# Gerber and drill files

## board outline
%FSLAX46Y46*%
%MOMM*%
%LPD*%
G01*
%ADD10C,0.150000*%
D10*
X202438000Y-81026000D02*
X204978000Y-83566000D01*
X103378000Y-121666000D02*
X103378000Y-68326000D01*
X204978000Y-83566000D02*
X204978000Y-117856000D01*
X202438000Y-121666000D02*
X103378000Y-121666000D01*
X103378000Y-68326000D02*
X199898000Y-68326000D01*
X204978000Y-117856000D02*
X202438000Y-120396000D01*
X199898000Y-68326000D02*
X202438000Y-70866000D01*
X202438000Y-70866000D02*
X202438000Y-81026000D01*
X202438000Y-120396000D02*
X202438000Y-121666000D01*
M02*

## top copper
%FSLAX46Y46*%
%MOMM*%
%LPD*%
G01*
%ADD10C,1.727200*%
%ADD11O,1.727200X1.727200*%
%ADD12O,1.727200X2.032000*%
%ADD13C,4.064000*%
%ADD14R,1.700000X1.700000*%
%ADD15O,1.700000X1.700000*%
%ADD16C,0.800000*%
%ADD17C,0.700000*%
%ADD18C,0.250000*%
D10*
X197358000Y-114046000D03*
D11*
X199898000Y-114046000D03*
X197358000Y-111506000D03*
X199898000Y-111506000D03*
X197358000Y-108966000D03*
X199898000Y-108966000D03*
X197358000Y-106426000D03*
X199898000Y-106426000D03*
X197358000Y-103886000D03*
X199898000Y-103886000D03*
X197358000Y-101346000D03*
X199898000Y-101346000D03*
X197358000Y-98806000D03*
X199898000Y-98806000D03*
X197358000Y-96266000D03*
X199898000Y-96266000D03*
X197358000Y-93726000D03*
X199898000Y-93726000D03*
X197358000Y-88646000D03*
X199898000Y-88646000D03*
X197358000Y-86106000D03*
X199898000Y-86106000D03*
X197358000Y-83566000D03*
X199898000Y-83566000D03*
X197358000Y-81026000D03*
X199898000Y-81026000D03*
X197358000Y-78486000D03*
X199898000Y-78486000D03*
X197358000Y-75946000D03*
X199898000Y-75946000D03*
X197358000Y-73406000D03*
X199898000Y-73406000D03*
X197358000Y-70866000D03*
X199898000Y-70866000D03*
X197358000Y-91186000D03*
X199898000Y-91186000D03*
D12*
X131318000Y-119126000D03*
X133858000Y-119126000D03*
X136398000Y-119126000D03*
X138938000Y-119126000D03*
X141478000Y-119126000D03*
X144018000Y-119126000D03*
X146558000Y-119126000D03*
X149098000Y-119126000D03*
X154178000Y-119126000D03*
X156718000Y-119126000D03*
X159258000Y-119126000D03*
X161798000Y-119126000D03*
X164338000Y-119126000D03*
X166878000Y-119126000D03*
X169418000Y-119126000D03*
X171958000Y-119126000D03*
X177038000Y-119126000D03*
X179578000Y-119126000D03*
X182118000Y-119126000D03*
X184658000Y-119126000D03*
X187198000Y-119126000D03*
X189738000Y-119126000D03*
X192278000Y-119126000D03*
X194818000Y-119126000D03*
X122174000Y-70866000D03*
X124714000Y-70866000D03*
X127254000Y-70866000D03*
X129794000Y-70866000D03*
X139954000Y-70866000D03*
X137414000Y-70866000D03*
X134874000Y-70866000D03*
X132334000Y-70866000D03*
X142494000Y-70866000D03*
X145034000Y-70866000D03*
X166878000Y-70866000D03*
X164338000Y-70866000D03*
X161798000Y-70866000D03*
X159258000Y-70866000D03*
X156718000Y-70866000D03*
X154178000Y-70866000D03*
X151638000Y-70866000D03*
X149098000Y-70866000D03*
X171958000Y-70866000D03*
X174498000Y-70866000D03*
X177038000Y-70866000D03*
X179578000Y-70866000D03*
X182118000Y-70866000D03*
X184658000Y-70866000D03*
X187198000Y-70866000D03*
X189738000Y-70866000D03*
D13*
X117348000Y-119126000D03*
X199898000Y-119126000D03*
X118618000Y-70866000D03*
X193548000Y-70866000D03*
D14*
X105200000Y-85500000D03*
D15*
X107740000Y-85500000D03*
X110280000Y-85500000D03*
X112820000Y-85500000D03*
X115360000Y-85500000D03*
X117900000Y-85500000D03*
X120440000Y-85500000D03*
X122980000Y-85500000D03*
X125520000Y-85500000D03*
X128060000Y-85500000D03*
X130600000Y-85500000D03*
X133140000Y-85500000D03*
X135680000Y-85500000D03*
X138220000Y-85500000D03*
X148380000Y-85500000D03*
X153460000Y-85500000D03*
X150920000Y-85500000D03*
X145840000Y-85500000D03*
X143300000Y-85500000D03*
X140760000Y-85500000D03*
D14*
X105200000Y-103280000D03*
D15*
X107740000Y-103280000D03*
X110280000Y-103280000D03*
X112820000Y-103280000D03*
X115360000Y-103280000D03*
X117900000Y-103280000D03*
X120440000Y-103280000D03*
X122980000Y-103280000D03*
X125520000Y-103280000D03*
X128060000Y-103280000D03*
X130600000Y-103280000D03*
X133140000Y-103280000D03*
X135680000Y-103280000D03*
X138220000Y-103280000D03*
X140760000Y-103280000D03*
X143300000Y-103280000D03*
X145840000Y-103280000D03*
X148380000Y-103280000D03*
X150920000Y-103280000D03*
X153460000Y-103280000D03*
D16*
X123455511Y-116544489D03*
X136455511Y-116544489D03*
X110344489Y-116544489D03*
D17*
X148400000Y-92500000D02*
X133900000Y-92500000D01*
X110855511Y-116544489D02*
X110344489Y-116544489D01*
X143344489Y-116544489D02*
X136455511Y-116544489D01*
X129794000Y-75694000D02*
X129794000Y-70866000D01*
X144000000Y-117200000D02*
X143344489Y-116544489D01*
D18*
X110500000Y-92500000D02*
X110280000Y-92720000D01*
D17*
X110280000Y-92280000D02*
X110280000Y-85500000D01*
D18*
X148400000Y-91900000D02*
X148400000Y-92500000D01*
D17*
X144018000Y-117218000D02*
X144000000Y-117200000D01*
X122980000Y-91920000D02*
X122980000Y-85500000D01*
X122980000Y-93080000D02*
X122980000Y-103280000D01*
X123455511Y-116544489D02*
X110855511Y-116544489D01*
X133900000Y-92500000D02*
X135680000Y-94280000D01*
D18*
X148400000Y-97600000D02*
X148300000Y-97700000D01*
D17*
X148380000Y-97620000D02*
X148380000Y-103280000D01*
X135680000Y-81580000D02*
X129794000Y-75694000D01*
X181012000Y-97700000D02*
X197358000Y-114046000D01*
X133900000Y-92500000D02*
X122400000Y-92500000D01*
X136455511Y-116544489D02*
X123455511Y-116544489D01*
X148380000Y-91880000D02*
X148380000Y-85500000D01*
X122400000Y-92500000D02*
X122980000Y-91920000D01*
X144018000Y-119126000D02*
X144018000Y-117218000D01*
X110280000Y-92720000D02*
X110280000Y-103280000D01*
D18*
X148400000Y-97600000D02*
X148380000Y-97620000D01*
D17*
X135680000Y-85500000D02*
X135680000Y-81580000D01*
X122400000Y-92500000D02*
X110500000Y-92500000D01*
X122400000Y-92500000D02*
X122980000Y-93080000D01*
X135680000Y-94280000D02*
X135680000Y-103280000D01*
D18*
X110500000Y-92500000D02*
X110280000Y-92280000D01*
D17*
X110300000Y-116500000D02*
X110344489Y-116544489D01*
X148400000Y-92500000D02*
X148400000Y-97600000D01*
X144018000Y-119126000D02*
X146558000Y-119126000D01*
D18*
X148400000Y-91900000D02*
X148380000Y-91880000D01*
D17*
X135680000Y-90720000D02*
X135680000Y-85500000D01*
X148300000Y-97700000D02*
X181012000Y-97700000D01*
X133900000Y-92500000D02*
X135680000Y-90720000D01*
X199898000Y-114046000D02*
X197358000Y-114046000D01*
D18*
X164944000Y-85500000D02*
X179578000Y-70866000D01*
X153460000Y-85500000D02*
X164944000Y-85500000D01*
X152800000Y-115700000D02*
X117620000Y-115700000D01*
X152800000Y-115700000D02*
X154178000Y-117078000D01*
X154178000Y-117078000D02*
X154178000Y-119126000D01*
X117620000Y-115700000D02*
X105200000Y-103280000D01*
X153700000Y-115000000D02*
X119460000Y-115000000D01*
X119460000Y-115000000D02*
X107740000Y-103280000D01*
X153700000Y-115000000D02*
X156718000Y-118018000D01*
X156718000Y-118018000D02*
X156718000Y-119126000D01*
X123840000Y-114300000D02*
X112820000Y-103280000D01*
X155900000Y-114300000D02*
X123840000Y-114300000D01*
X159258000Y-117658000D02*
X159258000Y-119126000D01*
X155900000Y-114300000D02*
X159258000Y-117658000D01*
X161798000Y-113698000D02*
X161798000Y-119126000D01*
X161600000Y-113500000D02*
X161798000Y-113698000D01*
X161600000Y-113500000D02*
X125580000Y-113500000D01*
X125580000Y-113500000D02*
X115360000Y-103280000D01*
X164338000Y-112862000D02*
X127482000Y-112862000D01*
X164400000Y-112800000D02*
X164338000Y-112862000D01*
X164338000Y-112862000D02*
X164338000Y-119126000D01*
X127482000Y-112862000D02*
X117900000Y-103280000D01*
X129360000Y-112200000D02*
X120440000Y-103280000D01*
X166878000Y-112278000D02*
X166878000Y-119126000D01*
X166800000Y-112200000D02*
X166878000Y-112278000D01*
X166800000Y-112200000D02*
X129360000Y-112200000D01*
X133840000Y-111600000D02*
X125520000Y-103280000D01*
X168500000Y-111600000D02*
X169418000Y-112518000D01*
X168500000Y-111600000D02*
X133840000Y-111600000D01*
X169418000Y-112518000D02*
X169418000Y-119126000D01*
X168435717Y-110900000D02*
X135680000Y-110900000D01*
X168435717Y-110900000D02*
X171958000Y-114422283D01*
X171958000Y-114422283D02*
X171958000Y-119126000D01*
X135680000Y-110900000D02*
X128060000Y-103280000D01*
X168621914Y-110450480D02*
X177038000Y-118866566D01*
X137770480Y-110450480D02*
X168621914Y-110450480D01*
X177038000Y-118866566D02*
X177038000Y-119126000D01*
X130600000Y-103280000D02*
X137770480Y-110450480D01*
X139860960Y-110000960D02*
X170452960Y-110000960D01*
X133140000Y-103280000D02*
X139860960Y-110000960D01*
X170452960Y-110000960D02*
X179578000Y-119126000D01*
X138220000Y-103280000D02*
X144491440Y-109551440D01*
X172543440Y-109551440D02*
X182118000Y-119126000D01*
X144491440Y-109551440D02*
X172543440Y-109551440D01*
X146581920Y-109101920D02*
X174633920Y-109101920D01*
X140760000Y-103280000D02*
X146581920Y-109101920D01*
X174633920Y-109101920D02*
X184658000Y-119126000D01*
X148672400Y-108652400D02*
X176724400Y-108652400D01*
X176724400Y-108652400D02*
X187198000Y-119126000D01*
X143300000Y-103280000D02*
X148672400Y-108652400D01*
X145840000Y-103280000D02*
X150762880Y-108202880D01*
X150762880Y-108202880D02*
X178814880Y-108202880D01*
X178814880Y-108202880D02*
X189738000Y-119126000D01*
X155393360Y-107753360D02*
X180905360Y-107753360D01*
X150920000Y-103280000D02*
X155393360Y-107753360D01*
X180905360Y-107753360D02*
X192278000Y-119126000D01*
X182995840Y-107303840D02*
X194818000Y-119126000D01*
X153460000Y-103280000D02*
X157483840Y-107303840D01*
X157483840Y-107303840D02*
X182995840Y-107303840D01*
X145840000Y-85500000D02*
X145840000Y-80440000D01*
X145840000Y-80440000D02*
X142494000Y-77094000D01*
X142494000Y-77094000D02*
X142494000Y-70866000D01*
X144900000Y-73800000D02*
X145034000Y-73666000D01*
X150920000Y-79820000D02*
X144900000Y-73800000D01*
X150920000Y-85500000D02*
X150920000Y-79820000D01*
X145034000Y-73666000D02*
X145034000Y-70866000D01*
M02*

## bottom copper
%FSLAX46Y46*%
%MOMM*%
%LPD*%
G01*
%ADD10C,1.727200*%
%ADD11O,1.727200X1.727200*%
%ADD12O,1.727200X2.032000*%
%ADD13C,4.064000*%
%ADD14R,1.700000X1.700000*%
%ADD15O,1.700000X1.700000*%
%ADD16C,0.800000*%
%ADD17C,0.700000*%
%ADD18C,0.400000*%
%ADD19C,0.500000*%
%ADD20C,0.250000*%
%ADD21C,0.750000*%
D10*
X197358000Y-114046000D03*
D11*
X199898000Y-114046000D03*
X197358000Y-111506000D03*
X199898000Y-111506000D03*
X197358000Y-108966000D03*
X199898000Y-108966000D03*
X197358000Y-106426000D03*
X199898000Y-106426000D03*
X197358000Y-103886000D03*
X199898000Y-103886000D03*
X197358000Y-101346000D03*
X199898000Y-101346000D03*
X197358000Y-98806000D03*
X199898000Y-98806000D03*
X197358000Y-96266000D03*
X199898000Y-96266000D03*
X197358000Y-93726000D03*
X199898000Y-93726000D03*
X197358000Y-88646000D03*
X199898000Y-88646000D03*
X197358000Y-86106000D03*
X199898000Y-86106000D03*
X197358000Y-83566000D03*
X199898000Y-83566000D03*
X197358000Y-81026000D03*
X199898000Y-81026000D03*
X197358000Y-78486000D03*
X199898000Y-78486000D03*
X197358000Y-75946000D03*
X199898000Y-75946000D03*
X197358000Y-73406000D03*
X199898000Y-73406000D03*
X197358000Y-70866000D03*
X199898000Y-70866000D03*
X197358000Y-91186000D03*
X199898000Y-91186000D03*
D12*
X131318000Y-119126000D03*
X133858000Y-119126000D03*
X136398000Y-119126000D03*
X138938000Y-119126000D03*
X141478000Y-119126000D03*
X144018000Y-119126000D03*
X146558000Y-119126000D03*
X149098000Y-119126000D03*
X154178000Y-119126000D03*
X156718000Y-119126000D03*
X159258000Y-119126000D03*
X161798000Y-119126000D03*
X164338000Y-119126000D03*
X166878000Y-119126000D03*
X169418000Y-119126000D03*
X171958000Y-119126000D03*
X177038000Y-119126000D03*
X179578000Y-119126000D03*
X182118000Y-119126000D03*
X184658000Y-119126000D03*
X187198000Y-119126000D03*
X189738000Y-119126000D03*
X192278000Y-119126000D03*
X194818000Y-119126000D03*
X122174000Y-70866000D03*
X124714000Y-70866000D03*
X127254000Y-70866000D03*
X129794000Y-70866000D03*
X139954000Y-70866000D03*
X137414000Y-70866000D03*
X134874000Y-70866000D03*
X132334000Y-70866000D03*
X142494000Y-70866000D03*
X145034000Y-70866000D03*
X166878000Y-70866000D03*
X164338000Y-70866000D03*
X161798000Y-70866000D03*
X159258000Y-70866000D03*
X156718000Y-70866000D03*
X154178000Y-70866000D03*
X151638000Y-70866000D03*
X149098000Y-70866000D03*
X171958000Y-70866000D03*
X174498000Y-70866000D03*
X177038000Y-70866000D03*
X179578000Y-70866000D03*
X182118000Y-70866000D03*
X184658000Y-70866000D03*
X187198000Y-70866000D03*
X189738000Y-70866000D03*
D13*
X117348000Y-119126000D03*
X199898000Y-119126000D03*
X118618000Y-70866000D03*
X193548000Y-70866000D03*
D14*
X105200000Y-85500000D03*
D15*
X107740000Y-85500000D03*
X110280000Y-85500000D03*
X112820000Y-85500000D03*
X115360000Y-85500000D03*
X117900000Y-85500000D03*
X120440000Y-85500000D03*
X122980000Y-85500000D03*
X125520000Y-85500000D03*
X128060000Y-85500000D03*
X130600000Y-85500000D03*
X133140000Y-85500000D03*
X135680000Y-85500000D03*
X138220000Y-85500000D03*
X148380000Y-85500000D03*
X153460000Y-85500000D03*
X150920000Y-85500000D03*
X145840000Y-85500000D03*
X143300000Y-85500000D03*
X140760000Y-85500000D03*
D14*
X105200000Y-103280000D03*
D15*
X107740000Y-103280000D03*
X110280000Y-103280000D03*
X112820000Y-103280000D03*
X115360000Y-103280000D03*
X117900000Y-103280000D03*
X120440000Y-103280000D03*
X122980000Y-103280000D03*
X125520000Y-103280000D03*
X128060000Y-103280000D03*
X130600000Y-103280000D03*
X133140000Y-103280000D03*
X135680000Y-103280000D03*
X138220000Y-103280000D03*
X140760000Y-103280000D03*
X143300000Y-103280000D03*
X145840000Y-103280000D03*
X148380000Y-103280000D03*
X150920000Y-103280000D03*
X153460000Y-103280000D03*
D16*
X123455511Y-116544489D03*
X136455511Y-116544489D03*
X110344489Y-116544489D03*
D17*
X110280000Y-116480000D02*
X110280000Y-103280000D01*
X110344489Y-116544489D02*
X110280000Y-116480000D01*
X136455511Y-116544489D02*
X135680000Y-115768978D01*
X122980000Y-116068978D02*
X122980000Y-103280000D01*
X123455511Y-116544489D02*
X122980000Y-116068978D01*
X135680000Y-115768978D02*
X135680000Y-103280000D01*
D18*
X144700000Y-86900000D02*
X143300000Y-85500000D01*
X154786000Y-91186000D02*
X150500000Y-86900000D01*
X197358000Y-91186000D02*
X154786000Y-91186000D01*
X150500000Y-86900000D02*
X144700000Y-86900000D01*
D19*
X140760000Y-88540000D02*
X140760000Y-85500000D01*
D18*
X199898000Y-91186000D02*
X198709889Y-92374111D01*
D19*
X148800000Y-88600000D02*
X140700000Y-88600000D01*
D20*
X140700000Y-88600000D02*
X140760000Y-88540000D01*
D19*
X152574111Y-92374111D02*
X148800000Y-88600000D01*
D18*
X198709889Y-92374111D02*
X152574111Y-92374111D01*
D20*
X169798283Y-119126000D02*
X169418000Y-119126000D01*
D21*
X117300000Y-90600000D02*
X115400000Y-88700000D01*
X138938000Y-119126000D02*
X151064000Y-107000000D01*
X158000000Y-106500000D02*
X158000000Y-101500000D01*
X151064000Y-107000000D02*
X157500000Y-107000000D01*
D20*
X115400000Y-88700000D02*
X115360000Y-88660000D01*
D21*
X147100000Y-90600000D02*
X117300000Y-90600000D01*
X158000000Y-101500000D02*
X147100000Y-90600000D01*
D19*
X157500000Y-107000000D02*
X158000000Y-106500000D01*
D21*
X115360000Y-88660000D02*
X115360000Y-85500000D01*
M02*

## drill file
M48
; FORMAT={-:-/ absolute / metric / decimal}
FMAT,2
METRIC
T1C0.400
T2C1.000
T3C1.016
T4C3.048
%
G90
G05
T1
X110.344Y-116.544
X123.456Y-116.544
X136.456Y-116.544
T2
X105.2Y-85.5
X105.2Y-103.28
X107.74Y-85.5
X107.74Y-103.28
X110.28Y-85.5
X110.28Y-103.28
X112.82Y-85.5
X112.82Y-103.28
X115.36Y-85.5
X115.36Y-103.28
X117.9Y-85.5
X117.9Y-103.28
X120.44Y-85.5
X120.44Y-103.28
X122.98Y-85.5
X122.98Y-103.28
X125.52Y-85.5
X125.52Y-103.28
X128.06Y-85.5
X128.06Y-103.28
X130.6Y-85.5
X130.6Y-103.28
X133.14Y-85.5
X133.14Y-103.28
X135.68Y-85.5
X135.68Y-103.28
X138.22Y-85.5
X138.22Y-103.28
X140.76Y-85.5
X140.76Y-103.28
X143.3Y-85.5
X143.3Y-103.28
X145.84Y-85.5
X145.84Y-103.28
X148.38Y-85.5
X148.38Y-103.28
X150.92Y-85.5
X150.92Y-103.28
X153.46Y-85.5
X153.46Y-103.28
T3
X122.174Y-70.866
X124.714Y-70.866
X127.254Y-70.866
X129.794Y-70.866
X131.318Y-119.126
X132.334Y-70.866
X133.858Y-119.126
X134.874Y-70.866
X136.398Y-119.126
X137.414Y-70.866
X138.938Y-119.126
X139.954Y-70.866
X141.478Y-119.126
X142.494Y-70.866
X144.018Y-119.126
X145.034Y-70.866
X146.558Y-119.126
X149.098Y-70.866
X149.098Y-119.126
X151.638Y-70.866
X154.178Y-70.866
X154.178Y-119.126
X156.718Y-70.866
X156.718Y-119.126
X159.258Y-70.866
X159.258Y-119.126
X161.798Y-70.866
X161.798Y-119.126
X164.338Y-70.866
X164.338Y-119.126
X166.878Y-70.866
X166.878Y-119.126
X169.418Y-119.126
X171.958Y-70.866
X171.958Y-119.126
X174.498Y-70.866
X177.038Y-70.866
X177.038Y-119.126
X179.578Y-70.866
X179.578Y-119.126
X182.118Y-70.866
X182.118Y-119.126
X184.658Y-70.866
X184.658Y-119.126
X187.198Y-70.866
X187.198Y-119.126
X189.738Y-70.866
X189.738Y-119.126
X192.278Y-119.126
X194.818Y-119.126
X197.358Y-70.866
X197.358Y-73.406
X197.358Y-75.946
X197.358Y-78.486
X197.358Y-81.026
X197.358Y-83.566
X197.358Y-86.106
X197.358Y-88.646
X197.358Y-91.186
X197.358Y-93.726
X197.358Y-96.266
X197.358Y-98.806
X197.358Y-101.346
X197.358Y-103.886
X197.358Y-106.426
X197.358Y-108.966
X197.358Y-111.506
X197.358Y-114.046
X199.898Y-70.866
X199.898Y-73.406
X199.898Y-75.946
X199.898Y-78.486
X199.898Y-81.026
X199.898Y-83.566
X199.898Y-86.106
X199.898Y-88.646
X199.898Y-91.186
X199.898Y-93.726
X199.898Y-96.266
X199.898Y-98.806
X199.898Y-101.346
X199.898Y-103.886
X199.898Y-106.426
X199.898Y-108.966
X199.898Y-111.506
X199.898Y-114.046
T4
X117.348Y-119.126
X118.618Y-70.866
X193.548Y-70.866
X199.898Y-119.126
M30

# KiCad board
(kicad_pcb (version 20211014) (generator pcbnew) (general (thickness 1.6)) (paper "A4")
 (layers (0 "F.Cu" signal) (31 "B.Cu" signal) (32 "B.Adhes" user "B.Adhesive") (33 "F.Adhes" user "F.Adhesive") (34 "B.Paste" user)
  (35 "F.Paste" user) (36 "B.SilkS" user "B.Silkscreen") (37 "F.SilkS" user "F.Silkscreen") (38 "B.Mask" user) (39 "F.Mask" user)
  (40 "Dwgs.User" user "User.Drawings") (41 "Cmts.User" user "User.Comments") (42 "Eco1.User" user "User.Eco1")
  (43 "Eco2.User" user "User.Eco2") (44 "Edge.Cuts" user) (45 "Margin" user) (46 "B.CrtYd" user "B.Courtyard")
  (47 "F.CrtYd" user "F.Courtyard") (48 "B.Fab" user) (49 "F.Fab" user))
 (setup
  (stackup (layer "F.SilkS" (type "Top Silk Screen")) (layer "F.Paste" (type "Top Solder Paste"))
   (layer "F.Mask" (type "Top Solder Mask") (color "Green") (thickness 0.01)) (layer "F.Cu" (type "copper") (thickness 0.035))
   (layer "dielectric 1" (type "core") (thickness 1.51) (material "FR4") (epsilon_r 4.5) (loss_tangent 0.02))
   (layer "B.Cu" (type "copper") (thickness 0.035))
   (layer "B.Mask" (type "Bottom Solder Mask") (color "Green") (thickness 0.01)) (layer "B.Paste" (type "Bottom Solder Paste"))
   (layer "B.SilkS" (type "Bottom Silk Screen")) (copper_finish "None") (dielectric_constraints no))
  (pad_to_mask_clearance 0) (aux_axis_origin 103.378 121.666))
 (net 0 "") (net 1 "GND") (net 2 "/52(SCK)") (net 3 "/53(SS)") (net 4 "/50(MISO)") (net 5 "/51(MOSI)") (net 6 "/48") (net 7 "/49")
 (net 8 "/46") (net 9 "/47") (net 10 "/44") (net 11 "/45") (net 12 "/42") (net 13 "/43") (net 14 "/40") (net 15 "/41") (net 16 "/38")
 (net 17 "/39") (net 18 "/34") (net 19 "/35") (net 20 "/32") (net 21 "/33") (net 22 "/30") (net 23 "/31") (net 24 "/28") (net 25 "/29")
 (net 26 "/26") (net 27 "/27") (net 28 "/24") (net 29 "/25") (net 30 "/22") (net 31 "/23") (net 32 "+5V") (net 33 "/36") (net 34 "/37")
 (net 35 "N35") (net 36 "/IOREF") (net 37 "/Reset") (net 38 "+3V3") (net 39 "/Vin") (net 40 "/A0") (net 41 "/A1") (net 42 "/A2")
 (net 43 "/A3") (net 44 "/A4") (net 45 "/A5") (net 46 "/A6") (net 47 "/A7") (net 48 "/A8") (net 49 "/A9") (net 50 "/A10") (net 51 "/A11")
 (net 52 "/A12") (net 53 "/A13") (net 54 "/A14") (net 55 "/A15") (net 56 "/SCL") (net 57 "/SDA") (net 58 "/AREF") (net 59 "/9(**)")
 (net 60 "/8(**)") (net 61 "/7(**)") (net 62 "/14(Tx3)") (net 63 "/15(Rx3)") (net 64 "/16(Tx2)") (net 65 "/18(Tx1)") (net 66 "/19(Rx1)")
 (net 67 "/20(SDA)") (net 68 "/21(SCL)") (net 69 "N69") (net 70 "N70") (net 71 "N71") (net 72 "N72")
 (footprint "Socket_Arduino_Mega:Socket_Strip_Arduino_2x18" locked (layer "F.Cu") (at 197.358 114.046 90)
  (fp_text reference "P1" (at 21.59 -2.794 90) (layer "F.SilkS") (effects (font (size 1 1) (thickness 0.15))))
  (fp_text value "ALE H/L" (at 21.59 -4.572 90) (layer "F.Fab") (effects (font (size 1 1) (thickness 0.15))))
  (pad "1" thru_hole circle locked (at 0 0 90) (size 1.7272 1.7272) (drill 1.016) (layers *.Cu *.Mask "F.SilkS") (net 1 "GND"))
  (pad "2" thru_hole oval locked (at 0 2.54 90) (size 1.7272 1.7272) (drill 1.016) (layers *.Cu *.Mask "F.SilkS") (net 1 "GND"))
  (pad "3" thru_hole oval locked (at 2.54 0 90) (size 1.7272 1.7272) (drill 1.016) (layers *.Cu *.Mask "F.SilkS") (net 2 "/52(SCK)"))
  (pad "4" thru_hole oval locked (at 2.54 2.54 90) (size 1.7272 1.7272) (drill 1.016) (layers *.Cu *.Mask "F.SilkS") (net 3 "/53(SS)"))
  (pad "5" thru_hole oval locked (at 5.08 0 90) (size 1.7272 1.7272) (drill 1.016) (layers *.Cu *.Mask "F.SilkS") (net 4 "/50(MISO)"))
  (pad "6" thru_hole oval locked (at 5.08 2.54 90) (size 1.7272 1.7272) (drill 1.016) (layers *.Cu *.Mask "F.SilkS") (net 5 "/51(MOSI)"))
  (pad "7" thru_hole oval locked (at 7.62 0 90) (size 1.7272 1.7272) (drill 1.016) (layers *.Cu *.Mask "F.SilkS") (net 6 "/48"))
  (pad "8" thru_hole oval locked (at 7.62 2.54 90) (size 1.7272 1.7272) (drill 1.016) (layers *.Cu *.Mask "F.SilkS") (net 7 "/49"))
  (pad "9" thru_hole oval locked (at 10.16 0 90) (size 1.7272 1.7272) (drill 1.016) (layers *.Cu *.Mask "F.SilkS") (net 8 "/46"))
  (pad "10" thru_hole oval locked (at 10.16 2.54 90) (size 1.7272 1.7272) (drill 1.016) (layers *.Cu *.Mask "F.SilkS") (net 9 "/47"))
  (pad "11" thru_hole oval locked (at 12.7 0 90) (size 1.7272 1.7272) (drill 1.016) (layers *.Cu *.Mask "F.SilkS") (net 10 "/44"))
  (pad "12" thru_hole oval locked (at 12.7 2.54 90) (size 1.7272 1.7272) (drill 1.016) (layers *.Cu *.Mask "F.SilkS") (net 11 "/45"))
  (pad "13" thru_hole oval locked (at 15.24 0 90) (size 1.7272 1.7272) (drill 1.016) (layers *.Cu *.Mask "F.SilkS") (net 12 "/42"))
  (pad "14" thru_hole oval locked (at 15.24 2.54 90) (size 1.7272 1.7272) (drill 1.016) (layers *.Cu *.Mask "F.SilkS") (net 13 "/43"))
  (pad "15" thru_hole oval locked (at 17.78 0 90) (size 1.7272 1.7272) (drill 1.016) (layers *.Cu *.Mask "F.SilkS") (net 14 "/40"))
  (pad "16" thru_hole oval locked (at 17.78 2.54 90) (size 1.7272 1.7272) (drill 1.016) (layers *.Cu *.Mask "F.SilkS") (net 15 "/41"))
  (pad "17" thru_hole oval locked (at 20.32 0 90) (size 1.7272 1.7272) (drill 1.016) (layers *.Cu *.Mask "F.SilkS") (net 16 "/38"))
  (pad "18" thru_hole oval locked (at 20.32 2.54 90) (size 1.7272 1.7272) (drill 1.016) (layers *.Cu *.Mask "F.SilkS") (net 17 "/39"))
  (pad "21" thru_hole oval locked (at 25.4 0 90) (size 1.7272 1.7272) (drill 1.016) (layers *.Cu *.Mask "F.SilkS") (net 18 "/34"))
  (pad "22" thru_hole oval locked (at 25.4 2.54 90) (size 1.7272 1.7272) (drill 1.016) (layers *.Cu *.Mask "F.SilkS") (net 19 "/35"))
  (pad "23" thru_hole oval locked (at 27.94 0 90) (size 1.7272 1.7272) (drill 1.016) (layers *.Cu *.Mask "F.SilkS") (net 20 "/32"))
  (pad "24" thru_hole oval locked (at 27.94 2.54 90) (size 1.7272 1.7272) (drill 1.016) (layers *.Cu *.Mask "F.SilkS") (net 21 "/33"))
  (pad "25" thru_hole oval locked (at 30.48 0 90) (size 1.7272 1.7272) (drill 1.016) (layers *.Cu *.Mask "F.SilkS") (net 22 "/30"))
  (pad "26" thru_hole oval locked (at 30.48 2.54 90) (size 1.7272 1.7272) (drill 1.016) (layers *.Cu *.Mask "F.SilkS") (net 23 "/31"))
  (pad "27" thru_hole oval locked (at 33.02 0 90) (size 1.7272 1.7272) (drill 1.016) (layers *.Cu *.Mask "F.SilkS") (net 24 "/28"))
  (pad "28" thru_hole oval locked (at 33.02 2.54 90) (size 1.7272 1.7272) (drill 1.016) (layers *.Cu *.Mask "F.SilkS") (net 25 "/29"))
  (pad "29" thru_hole oval locked (at 35.56 0 90) (size 1.7272 1.7272) (drill 1.016) (layers *.Cu *.Mask "F.SilkS") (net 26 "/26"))
  (pad "30" thru_hole oval locked (at 35.56 2.54 90) (size 1.7272 1.7272) (drill 1.016) (layers *.Cu *.Mask "F.SilkS") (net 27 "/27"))
  (pad "31" thru_hole oval locked (at 38.1 0 90) (size 1.7272 1.7272) (drill 1.016) (layers *.Cu *.Mask "F.SilkS") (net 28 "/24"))
  (pad "32" thru_hole oval locked (at 38.1 2.54 90) (size 1.7272 1.7272) (drill 1.016) (layers *.Cu *.Mask "F.SilkS") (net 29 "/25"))
  (pad "33" thru_hole oval locked (at 40.64 0 90) (size 1.7272 1.7272) (drill 1.016) (layers *.Cu *.Mask "F.SilkS") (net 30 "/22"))
  (pad "34" thru_hole oval locked (at 40.64 2.54 90) (size 1.7272 1.7272) (drill 1.016) (layers *.Cu *.Mask "F.SilkS") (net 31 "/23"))
  (pad "35" thru_hole oval locked (at 43.18 0 90) (size 1.7272 1.7272) (drill 1.016) (layers *.Cu *.Mask "F.SilkS") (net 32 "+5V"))
  (pad "36" thru_hole oval locked (at 43.18 2.54 90) (size 1.7272 1.7272) (drill 1.016) (layers *.Cu *.Mask "F.SilkS") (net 32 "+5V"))
  (pad "36" thru_hole oval locked (at 22.86 0 90) (size 1.7272 1.7272) (drill 1.016) (layers *.Cu *.Mask "F.SilkS") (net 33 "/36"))
  (pad "37" thru_hole oval locked (at 22.86 2.54 90) (size 1.7272 1.7272) (drill 1.016) (layers *.Cu *.Mask "F.SilkS") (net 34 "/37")))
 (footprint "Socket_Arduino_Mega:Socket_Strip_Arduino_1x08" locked (layer "F.Cu") (at 131.318 119.126)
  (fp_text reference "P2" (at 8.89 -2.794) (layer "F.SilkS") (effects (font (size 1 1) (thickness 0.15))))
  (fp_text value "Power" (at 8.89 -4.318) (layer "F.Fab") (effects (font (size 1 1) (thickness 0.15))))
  (pad "1" thru_hole oval locked (at 0 0) (size 1.7272 2.032) (drill 1.016) (layers *.Cu *.Mask "F.SilkS") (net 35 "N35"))
  (pad "2" thru_hole oval locked (at 2.54 0) (size 1.7272 2.032) (drill 1.016) (layers *.Cu *.Mask "F.SilkS") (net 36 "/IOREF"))
  (pad "3" thru_hole oval locked (at 5.08 0) (size 1.7272 2.032) (drill 1.016) (layers *.Cu *.Mask "F.SilkS") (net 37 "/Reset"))
  (pad "4" thru_hole oval locked (at 7.62 0) (size 1.7272 2.032) (drill 1.016) (layers *.Cu *.Mask "F.SilkS") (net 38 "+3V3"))
  (pad "5" thru_hole oval locked (at 10.16 0) (size 1.7272 2.032) (drill 1.016) (layers *.Cu *.Mask "F.SilkS") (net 32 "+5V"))
  (pad "6" thru_hole oval locked (at 12.7 0) (size 1.7272 2.032) (drill 1.016) (layers *.Cu *.Mask "F.SilkS") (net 1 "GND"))
  (pad "7" thru_hole oval locked (at 15.24 0) (size 1.7272 2.032) (drill 1.016) (layers *.Cu *.Mask "F.SilkS") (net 1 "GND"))
  (pad "8" thru_hole oval locked (at 17.78 0) (size 1.7272 2.032) (drill 1.016) (layers *.Cu *.Mask "F.SilkS") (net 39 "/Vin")))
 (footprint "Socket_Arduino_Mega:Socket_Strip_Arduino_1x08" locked (layer "F.Cu") (at 154.178 119.126)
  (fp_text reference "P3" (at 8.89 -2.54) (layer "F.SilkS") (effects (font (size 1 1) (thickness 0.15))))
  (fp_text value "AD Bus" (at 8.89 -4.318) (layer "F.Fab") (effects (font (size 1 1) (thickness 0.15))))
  (pad "1" thru_hole oval locked (at 0 0) (size 1.7272 2.032) (drill 1.016) (layers *.Cu *.Mask "F.SilkS") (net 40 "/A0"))
  (pad "2" thru_hole oval locked (at 2.54 0) (size 1.7272 2.032) (drill 1.016) (layers *.Cu *.Mask "F.SilkS") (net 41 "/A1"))
  (pad "3" thru_hole oval locked (at 5.08 0) (size 1.7272 2.032) (drill 1.016) (layers *.Cu *.Mask "F.SilkS") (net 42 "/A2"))
  (pad "4" thru_hole oval locked (at 7.62 0) (size 1.7272 2.032) (drill 1.016) (layers *.Cu *.Mask "F.SilkS") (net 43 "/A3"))
  (pad "5" thru_hole oval locked (at 10.16 0) (size 1.7272 2.032) (drill 1.016) (layers *.Cu *.Mask "F.SilkS") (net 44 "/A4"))
  (pad "6" thru_hole oval locked (at 12.7 0) (size 1.7272 2.032) (drill 1.016) (layers *.Cu *.Mask "F.SilkS") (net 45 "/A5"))
  (pad "7" thru_hole oval locked (at 15.24 0) (size 1.7272 2.032) (drill 1.016) (layers *.Cu *.Mask "F.SilkS") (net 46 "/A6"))
  (pad "8" thru_hole oval locked (at 17.78 0) (size 1.7272 2.032) (drill 1.016) (layers *.Cu *.Mask "F.SilkS") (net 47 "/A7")))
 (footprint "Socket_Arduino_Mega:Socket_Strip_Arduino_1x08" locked (layer "F.Cu") (at 177.038 119.126)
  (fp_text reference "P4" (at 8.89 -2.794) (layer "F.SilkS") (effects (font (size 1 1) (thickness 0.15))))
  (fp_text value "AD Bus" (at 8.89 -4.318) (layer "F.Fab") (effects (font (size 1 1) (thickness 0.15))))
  (pad "1" thru_hole oval locked (at 0 0) (size 1.7272 2.032) (drill 1.016) (layers *.Cu *.Mask "F.SilkS") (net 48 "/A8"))
  (pad "2" thru_hole oval locked (at 2.54 0) (size 1.7272 2.032) (drill 1.016) (layers *.Cu *.Mask "F.SilkS") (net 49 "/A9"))
  (pad "3" thru_hole oval locked (at 5.08 0) (size 1.7272 2.032) (drill 1.016) (layers *.Cu *.Mask "F.SilkS") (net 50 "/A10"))
  (pad "4" thru_hole oval locked (at 7.62 0) (size 1.7272 2.032) (drill 1.016) (layers *.Cu *.Mask "F.SilkS") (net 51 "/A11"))
  (pad "5" thru_hole oval locked (at 10.16 0) (size 1.7272 2.032) (drill 1.016) (layers *.Cu *.Mask "F.SilkS") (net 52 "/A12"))
  (pad "6" thru_hole oval locked (at 12.7 0) (size 1.7272 2.032) (drill 1.016) (layers *.Cu *.Mask "F.SilkS") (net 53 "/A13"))
  (pad "7" thru_hole oval locked (at 15.24 0) (size 1.7272 2.032) (drill 1.016) (layers *.Cu *.Mask "F.SilkS") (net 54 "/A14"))
  (pad "8" thru_hole oval locked (at 17.78 0) (size 1.7272 2.032) (drill 1.016) (layers *.Cu *.Mask "F.SilkS") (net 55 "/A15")))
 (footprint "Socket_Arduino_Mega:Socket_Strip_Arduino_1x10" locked (layer "F.Cu") (at 122.174 70.866)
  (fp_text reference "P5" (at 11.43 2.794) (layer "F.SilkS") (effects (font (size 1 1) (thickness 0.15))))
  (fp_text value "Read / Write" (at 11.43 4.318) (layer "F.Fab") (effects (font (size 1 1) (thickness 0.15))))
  (pad "1" thru_hole oval locked (at 0 0) (size 1.7272 2.032) (drill 1.016) (layers *.Cu *.Mask "F.SilkS") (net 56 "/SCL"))
  (pad "2" thru_hole oval locked (at 2.54 0) (size 1.7272 2.032) (drill 1.016) (layers *.Cu *.Mask "F.SilkS") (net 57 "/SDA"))
  (pad "3" thru_hole oval locked (at 5.08 0) (size 1.7272 2.032) (drill 1.016) (layers *.Cu *.Mask "F.SilkS") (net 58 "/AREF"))
  (pad "4" thru_hole oval locked (at 7.62 0) (size 1.7272 2.032) (drill 1.016) (layers *.Cu *.Mask "F.SilkS") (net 1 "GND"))
  (pad "10" thru_hole oval locked (at 17.78 0) (size 1.7272 2.032) (drill 1.016) (layers *.Cu *.Mask "F.SilkS"))
  (pad "11" thru_hole oval locked (at 15.24 0) (size 1.7272 2.032) (drill 1.016) (layers *.Cu *.Mask "F.SilkS"))
  (pad "12" thru_hole oval locked (at 12.7 0) (size 1.7272 2.032) (drill 1.016) (layers *.Cu *.Mask "F.SilkS"))
  (pad "13" thru_hole oval locked (at 10.16 0) (size 1.7272 2.032) (drill 1.016) (layers *.Cu *.Mask "F.SilkS"))
  (pad "READ" thru_hole oval locked (at 20.32 0) (size 1.7272 2.032) (drill 1.016) (layers *.Cu *.Mask "F.SilkS") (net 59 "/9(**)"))
  (pad "WRITE" thru_hole oval locked (at 22.86 0) (size 1.7272 2.032) (drill 1.016) (layers *.Cu *.Mask "F.SilkS") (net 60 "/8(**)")))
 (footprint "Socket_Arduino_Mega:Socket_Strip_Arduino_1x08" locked (layer "F.Cu") (at 149.098 70.866)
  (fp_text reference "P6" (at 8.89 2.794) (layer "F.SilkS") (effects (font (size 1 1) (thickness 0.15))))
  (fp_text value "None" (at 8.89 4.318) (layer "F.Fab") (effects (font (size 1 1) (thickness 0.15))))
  (pad "0" thru_hole oval locked (at 17.78 0) (size 1.7272 2.032) (drill 1.016) (layers *.Cu *.Mask "F.SilkS"))
  (pad "1" thru_hole oval locked (at 15.24 0) (size 1.7272 2.032) (drill 1.016) (layers *.Cu *.Mask "F.SilkS"))
  (pad "2" thru_hole oval locked (at 12.7 0) (size 1.7272 2.032) (drill 1.016) (layers *.Cu *.Mask "F.SilkS"))
  (pad "3" thru_hole oval locked (at 10.16 0) (size 1.7272 2.032) (drill 1.016) (layers *.Cu *.Mask "F.SilkS"))
  (pad "4" thru_hole oval locked (at 7.62 0) (size 1.7272 2.032) (drill 1.016) (layers *.Cu *.Mask "F.SilkS"))
  (pad "5" thru_hole oval locked (at 5.08 0) (size 1.7272 2.032) (drill 1.016) (layers *.Cu *.Mask "F.SilkS"))
  (pad "6" thru_hole oval locked (at 2.54 0) (size 1.7272 2.032) (drill 1.016) (layers *.Cu *.Mask "F.SilkS"))
  (pad "7" thru_hole oval locked (at 0 0) (size 1.7272 2.032) (drill 1.016) (layers *.Cu *.Mask "F.SilkS") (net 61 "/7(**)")))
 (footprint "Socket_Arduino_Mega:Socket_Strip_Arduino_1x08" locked (layer "F.Cu") (at 171.958 70.866)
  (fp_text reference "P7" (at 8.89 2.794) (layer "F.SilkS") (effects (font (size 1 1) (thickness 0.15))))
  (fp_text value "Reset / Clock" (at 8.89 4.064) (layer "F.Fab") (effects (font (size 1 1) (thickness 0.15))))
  (pad "14" thru_hole oval locked (at 0 0) (size 1.7272 2.032) (drill 1.016) (layers *.Cu *.Mask "F.SilkS") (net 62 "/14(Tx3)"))
  (pad "15" thru_hole oval locked (at 2.54 0) (size 1.7272 2.032) (drill 1.016) (layers *.Cu *.Mask "F.SilkS") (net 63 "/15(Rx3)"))
  (pad "16" thru_hole oval locked (at 5.08 0) (size 1.7272 2.032) (drill 1.016) (layers *.Cu *.Mask "F.SilkS") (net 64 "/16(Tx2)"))
  (pad "17" thru_hole oval locked (at 7.62 0) (size 1.7272 2.032) (drill 1.016) (layers *.Cu *.Mask "F.SilkS") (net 37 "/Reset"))
  (pad "18" thru_hole oval locked (at 10.16 0) (size 1.7272 2.032) (drill 1.016) (layers *.Cu *.Mask "F.SilkS") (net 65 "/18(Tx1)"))
  (pad "19" thru_hole oval locked (at 12.7 0) (size 1.7272 2.032) (drill 1.016) (layers *.Cu *.Mask "F.SilkS") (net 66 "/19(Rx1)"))
  (pad "20" thru_hole oval locked (at 15.24 0) (size 1.7272 2.032) (drill 1.016) (layers *.Cu *.Mask "F.SilkS") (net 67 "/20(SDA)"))
  (pad "21" thru_hole oval locked (at 17.78 0) (size 1.7272 2.032) (drill 1.016) (layers *.Cu *.Mask "F.SilkS") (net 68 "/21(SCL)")))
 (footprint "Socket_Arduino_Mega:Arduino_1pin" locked (layer "F.Cu") (at 117.348 119.126)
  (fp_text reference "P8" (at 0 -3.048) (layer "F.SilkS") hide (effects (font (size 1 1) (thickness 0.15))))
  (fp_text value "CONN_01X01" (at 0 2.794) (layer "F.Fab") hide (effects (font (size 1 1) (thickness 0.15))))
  (pad "1" thru_hole circle locked (at 0 0) (size 4.064 4.064) (drill 3.048) (layers *.Cu *.Mask "F.SilkS") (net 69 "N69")))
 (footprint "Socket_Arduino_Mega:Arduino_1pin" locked (layer "F.Cu") (at 199.898 119.126)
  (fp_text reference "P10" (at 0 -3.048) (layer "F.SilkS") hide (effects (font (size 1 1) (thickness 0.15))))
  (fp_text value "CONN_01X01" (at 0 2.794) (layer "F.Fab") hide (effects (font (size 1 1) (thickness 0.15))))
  (pad "1" thru_hole circle locked (at 0 0) (size 4.064 4.064) (drill 3.048) (layers *.Cu *.Mask "F.SilkS") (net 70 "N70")))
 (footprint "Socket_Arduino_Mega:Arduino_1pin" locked (layer "F.Cu") (at 118.618 70.866)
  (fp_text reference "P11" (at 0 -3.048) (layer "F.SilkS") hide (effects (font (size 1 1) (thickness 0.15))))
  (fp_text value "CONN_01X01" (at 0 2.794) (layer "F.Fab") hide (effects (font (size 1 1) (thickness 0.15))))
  (pad "1" thru_hole circle locked (at 0 0) (size 4.064 4.064) (drill 3.048) (layers *.Cu *.Mask "F.SilkS") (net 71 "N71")))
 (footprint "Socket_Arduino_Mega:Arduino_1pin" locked (layer "F.Cu") (at 193.548 70.866)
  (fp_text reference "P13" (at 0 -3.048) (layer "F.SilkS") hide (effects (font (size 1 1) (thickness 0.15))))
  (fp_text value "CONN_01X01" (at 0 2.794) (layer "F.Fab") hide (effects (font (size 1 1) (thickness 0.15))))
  (pad "1" thru_hole circle locked (at 0 0) (size 4.064 4.064) (drill 3.048) (layers *.Cu *.Mask "F.SilkS") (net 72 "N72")))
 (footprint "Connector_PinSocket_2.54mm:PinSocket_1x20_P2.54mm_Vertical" (layer "F.Cu") (at 105.2 85.5 90)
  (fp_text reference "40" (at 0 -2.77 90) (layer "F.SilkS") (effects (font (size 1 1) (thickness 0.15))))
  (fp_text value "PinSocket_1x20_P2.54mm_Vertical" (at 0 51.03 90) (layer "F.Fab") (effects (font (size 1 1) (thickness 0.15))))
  (pad "1" thru_hole rect (at 0 0 90) (size 1.7 1.7) (drill 1) (layers *.Cu *.Mask) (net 32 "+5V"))
  (pad "2" thru_hole oval (at 0 2.54 90) (size 1.7 1.7) (drill 1) (layers *.Cu *.Mask))
  (pad "3" thru_hole oval (at 0 5.08 90) (size 1.7 1.7) (drill 1) (layers *.Cu *.Mask) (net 1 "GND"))
  (pad "4" thru_hole oval (at 0 7.62 90) (size 1.7 1.7) (drill 1) (layers *.Cu *.Mask))
  (pad "5" thru_hole oval (at 0 10.16 90) (size 1.7 1.7) (drill 1) (layers *.Cu *.Mask) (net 38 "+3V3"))
  (pad "6" thru_hole oval (at 0 12.7 90) (size 1.7 1.7) (drill 1) (layers *.Cu *.Mask))
  (pad "7" thru_hole oval (at 0 15.24 90) (size 1.7 1.7) (drill 1) (layers *.Cu *.Mask))
  (pad "8" thru_hole oval (at 0 17.78 90) (size 1.7 1.7) (drill 1) (layers *.Cu *.Mask) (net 1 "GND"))
  (pad "9" thru_hole oval (at 0 20.32 90) (size 1.7 1.7) (drill 1) (layers *.Cu *.Mask))
  (pad "10" thru_hole oval (at 0 22.86 90) (size 1.7 1.7) (drill 1) (layers *.Cu *.Mask))
  (pad "11" thru_hole oval (at 0 25.4 90) (size 1.7 1.7) (drill 1) (layers *.Cu *.Mask))
  (pad "12" thru_hole oval (at 0 27.94 90) (size 1.7 1.7) (drill 1) (layers *.Cu *.Mask))
  (pad "13" thru_hole oval (at 0 30.48 90) (size 1.7 1.7) (drill 1) (layers *.Cu *.Mask) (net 1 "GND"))
  (pad "14" thru_hole oval (at 0 33.02 90) (size 1.7 1.7) (drill 1) (layers *.Cu *.Mask))
  (pad "18" thru_hole oval (at 0 43.18 90) (size 1.7 1.7) (drill 1) (layers *.Cu *.Mask) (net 1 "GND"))
  (pad "GPIO16" thru_hole oval (at 0 48.26 90) (size 1.7 1.7) (drill 1) (layers *.Cu *.Mask) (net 37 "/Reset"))
  (pad "GPIO17" thru_hole oval (at 0 45.72 90) (size 1.7 1.7) (drill 1) (layers *.Cu *.Mask) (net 60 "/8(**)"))
  (pad "GPIO18" thru_hole oval (at 0 40.64 90) (size 1.7 1.7) (drill 1) (layers *.Cu *.Mask) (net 59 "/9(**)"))
  (pad "GPIO19" thru_hole oval (at 0 38.1 90) (size 1.7 1.7) (drill 1) (layers *.Cu *.Mask) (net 33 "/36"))
  (pad "GPIO20" thru_hole oval (at 0 35.56 90) (size 1.7 1.7) (drill 1) (layers *.Cu *.Mask) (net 34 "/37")))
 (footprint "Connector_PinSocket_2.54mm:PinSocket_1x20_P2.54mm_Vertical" (layer "F.Cu") (at 105.2 103.28 90)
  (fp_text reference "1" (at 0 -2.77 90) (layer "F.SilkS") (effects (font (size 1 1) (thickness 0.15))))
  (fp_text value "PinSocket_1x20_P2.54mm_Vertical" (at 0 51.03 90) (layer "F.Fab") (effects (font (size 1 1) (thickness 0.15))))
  (pad "1" thru_hole rect (at 0 0 90) (size 1.7 1.7) (drill 1) (layers *.Cu *.Mask) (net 40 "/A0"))
  (pad "2" thru_hole oval (at 0 2.54 90) (size 1.7 1.7) (drill 1) (layers *.Cu *.Mask) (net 41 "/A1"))
  (pad "3" thru_hole oval (at 0 5.08 90) (size 1.7 1.7) (drill 1) (layers *.Cu *.Mask) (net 1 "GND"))
  (pad "4" thru_hole oval (at 0 7.62 90) (size 1.7 1.7) (drill 1) (layers *.Cu *.Mask) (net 42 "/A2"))
  (pad "5" thru_hole oval (at 0 10.16 90) (size 1.7 1.7) (drill 1) (layers *.Cu *.Mask) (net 43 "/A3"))
  (pad "6" thru_hole oval (at 0 12.7 90) (size 1.7 1.7) (drill 1) (layers *.Cu *.Mask) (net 44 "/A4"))
  (pad "7" thru_hole oval (at 0 15.24 90) (size 1.7 1.7) (drill 1) (layers *.Cu *.Mask) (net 45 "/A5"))
  (pad "8" thru_hole oval (at 0 17.78 90) (size 1.7 1.7) (drill 1) (layers *.Cu *.Mask) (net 1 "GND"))
  (pad "9" thru_hole oval (at 0 20.32 90) (size 1.7 1.7) (drill 1) (layers *.Cu *.Mask) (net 46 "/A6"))
  (pad "10" thru_hole oval (at 0 22.86 90) (size 1.7 1.7) (drill 1) (layers *.Cu *.Mask) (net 47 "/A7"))
  (pad "11" thru_hole oval (at 0 25.4 90) (size 1.7 1.7) (drill 1) (layers *.Cu *.Mask) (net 48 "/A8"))
  (pad "12" thru_hole oval (at 0 27.94 90) (size 1.7 1.7) (drill 1) (layers *.Cu *.Mask) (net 49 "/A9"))
  (pad "13" thru_hole oval (at 0 30.48 90) (size 1.7 1.7) (drill 1) (layers *.Cu *.Mask) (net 1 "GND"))
  (pad "14" thru_hole oval (at 0 33.02 90) (size 1.7 1.7) (drill 1) (layers *.Cu *.Mask) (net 50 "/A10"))
  (pad "15" thru_hole oval (at 0 35.56 90) (size 1.7 1.7) (drill 1) (layers *.Cu *.Mask) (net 51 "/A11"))
  (pad "16" thru_hole oval (at 0 38.1 90) (size 1.7 1.7) (drill 1) (layers *.Cu *.Mask) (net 52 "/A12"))
  (pad "17" thru_hole oval (at 0 40.64 90) (size 1.7 1.7) (drill 1) (layers *.Cu *.Mask) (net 53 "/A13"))
  (pad "18" thru_hole oval (at 0 43.18 90) (size 1.7 1.7) (drill 1) (layers *.Cu *.Mask) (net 1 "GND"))
  (pad "19" thru_hole oval (at 0 45.72 90) (size 1.7 1.7) (drill 1) (layers *.Cu *.Mask) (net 54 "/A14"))
  (pad "20" thru_hole oval (at 0 48.26 90) (size 1.7 1.7) (drill 1) (layers *.Cu *.Mask) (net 55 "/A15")))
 (gr_line (start 202.438 81.026) (end 204.978 83.566) (layer "Edge.Cuts") (width 0.15))
 (gr_line (start 103.378 121.666) (end 103.378 68.326) (layer "Edge.Cuts") (width 0.15))
 (gr_line (start 204.978 83.566) (end 204.978 117.856) (layer "Edge.Cuts") (width 0.15))
 (gr_line (start 202.438 121.666) (end 103.378 121.666) (layer "Edge.Cuts") (width 0.15))
 (gr_line (start 103.378 68.326) (end 199.898 68.326) (layer "Edge.Cuts") (width 0.15))
 (gr_line (start 204.978 117.856) (end 202.438 120.396) (layer "Edge.Cuts") (width 0.15))
 (gr_line (start 199.898 68.326) (end 202.438 70.866) (layer "Edge.Cuts") (width 0.15))
 (gr_line (start 202.438 70.866) (end 202.438 81.026) (layer "Edge.Cuts") (width 0.15))
 (gr_line (start 202.438 120.396) (end 202.438 121.666) (layer "Edge.Cuts") (width 0.15))
 (segment (start 148.4 92.5) (end 133.9 92.5) (width 0.7) (layer "F.Cu") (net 1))
 (segment (start 110.855511 116.544489) (end 110.344489 116.544489) (width 0.7) (layer "F.Cu") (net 1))
 (segment (start 143.344489 116.544489) (end 136.455511 116.544489) (width 0.7) (layer "F.Cu") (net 1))
 (segment (start 129.794 75.694) (end 129.794 70.866) (width 0.7) (layer "F.Cu") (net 1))
 (segment (start 144 117.2) (end 143.344489 116.544489) (width 0.7) (layer "F.Cu") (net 1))
 (segment (start 110.5 92.5) (end 110.28 92.72) (width 0.25) (layer "F.Cu") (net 1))
 (segment (start 110.28 92.28) (end 110.28 85.5) (width 0.7) (layer "F.Cu") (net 1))
 (segment (start 148.4 91.9) (end 148.4 92.5) (width 0.25) (layer "F.Cu") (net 1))
 (segment (start 144.018 117.218) (end 144 117.2) (width 0.7) (layer "F.Cu") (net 1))
 (segment (start 122.98 91.92) (end 122.98 85.5) (width 0.7) (layer "F.Cu") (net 1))
 (segment (start 122.98 93.08) (end 122.98 103.28) (width 0.7) (layer "F.Cu") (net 1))
 (segment (start 123.455511 116.544489) (end 110.855511 116.544489) (width 0.7) (layer "F.Cu") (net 1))
 (segment (start 133.9 92.5) (end 135.68 94.28) (width 0.7) (layer "F.Cu") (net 1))
 (segment (start 148.4 97.6) (end 148.3 97.7) (width 0.25) (layer "F.Cu") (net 1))
 (segment (start 148.38 97.62) (end 148.38 103.28) (width 0.7) (layer "F.Cu") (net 1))
 (segment (start 135.68 81.58) (end 129.794 75.694) (width 0.7) (layer "F.Cu") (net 1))
 (segment (start 181.012 97.7) (end 197.358 114.046) (width 0.7) (layer "F.Cu") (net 1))
 (segment (start 133.9 92.5) (end 122.4 92.5) (width 0.7) (layer "F.Cu") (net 1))
 (segment (start 136.455511 116.544489) (end 123.455511 116.544489) (width 0.7) (layer "F.Cu") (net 1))
 (segment (start 148.38 91.88) (end 148.38 85.5) (width 0.7) (layer "F.Cu") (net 1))
 (segment (start 122.4 92.5) (end 122.98 91.92) (width 0.7) (layer "F.Cu") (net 1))
 (segment (start 144.018 119.126) (end 144.018 117.218) (width 0.7) (layer "F.Cu") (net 1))
 (segment (start 110.28 92.72) (end 110.28 103.28) (width 0.7) (layer "F.Cu") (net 1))
 (segment (start 148.4 97.6) (end 148.38 97.62) (width 0.25) (layer "F.Cu") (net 1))
 (segment (start 135.68 85.5) (end 135.68 81.58) (width 0.7) (layer "F.Cu") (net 1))
 (segment (start 122.4 92.5) (end 110.5 92.5) (width 0.7) (layer "F.Cu") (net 1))
 (segment (start 122.4 92.5) (end 122.98 93.08) (width 0.7) (layer "F.Cu") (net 1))
 (segment (start 135.68 94.28) (end 135.68 103.28) (width 0.7) (layer "F.Cu") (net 1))
 (segment (start 110.5 92.5) (end 110.28 92.28) (width 0.25) (layer "F.Cu") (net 1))
 (segment (start 110.3 116.5) (end 110.344489 116.544489) (width 0.7) (layer "F.Cu") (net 1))
 (segment (start 148.4 92.5) (end 148.4 97.6) (width 0.7) (layer "F.Cu") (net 1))
 (segment (start 144.018 119.126) (end 146.558 119.126) (width 0.7) (layer "F.Cu") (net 1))
 (segment (start 148.4 91.9) (end 148.38 91.88) (width 0.25) (layer "F.Cu") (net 1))
 (segment (start 135.68 90.72) (end 135.68 85.5) (width 0.7) (layer "F.Cu") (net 1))
 (segment (start 148.3 97.7) (end 181.012 97.7) (width 0.7) (layer "F.Cu") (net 1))
 (segment (start 133.9 92.5) (end 135.68 90.72) (width 0.7) (layer "F.Cu") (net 1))
 (segment (start 199.898 114.046) (end 197.358 114.046) (width 0.7) (layer "F.Cu") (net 1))
 (via (at 123.455511 116.544489) (size 0.8) (drill 0.4) (layers "F.Cu" "B.Cu") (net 1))
 (via (at 136.455511 116.544489) (size 0.8) (drill 0.4) (layers "F.Cu" "B.Cu") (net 1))
 (via (at 110.344489 116.544489) (size 0.8) (drill 0.4) (layers "F.Cu" "B.Cu") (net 1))
 (segment (start 110.28 116.48) (end 110.28 103.28) (width 0.7) (layer "B.Cu") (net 1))
 (segment (start 110.344489 116.544489) (end 110.28 116.48) (width 0.7) (layer "B.Cu") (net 1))
 (segment (start 136.455511 116.544489) (end 135.68 115.768978) (width 0.7) (layer "B.Cu") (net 1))
 (segment (start 122.98 116.068978) (end 122.98 103.28) (width 0.7) (layer "B.Cu") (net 1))
 (segment (start 123.455511 116.544489) (end 122.98 116.068978) (width 0.7) (layer "B.Cu") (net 1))
 (segment (start 135.68 115.768978) (end 135.68 103.28) (width 0.7) (layer "B.Cu") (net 1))
 (segment (start 144.7 86.9) (end 143.3 85.5) (width 0.4) (layer "B.Cu") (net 33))
 (segment (start 154.786 91.186) (end 150.5 86.9) (width 0.4) (layer "B.Cu") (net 33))
 (segment (start 197.358 91.186) (end 154.786 91.186) (width 0.4) (layer "B.Cu") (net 33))
 (segment (start 150.5 86.9) (end 144.7 86.9) (width 0.4) (layer "B.Cu") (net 33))
 (segment (start 140.76 88.54) (end 140.76 85.5) (width 0.5) (layer "B.Cu") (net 34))
 (segment (start 199.898 91.186) (end 198.709889 92.374111) (width 0.4) (layer "B.Cu") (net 34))
 (segment (start 148.8 88.6) (end 140.7 88.6) (width 0.5) (layer "B.Cu") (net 34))
 (segment (start 140.7 88.6) (end 140.76 88.54) (width 0.25) (layer "B.Cu") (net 34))
 (segment (start 152.574111 92.374111) (end 148.8 88.6) (width 0.5) (layer "B.Cu") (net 34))
 (segment (start 198.709889 92.374111) (end 152.574111 92.374111) (width 0.4) (layer "B.Cu") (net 34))
 (segment (start 164.944 85.5) (end 179.578 70.866) (width 0.25) (layer "F.Cu") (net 37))
 (segment (start 153.46 85.5) (end 164.944 85.5) (width 0.25) (layer "F.Cu") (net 37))
 (segment (start 152.8 115.7) (end 117.62 115.7) (width 0.25) (layer "F.Cu") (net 40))
 (segment (start 152.8 115.7) (end 154.178 117.078) (width 0.25) (layer "F.Cu") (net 40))
 (segment (start 154.178 117.078) (end 154.178 119.126) (width 0.25) (layer "F.Cu") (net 40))
 (segment (start 117.62 115.7) (end 105.2 103.28) (width 0.25) (layer "F.Cu") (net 40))
 (segment (start 153.7 115) (end 119.46 115) (width 0.25) (layer "F.Cu") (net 41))
 (segment (start 119.46 115) (end 107.74 103.28) (width 0.25) (layer "F.Cu") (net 41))
 (segment (start 153.7 115) (end 156.718 118.018) (width 0.25) (layer "F.Cu") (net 41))
 (segment (start 156.718 118.018) (end 156.718 119.126) (width 0.25) (layer "F.Cu") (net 41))
 (segment (start 123.84 114.3) (end 112.82 103.28) (width 0.25) (layer "F.Cu") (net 42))
 (segment (start 155.9 114.3) (end 123.84 114.3) (width 0.25) (layer "F.Cu") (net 42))
 (segment (start 159.258 117.658) (end 159.258 119.126) (width 0.25) (layer "F.Cu") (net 42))
 (segment (start 155.9 114.3) (end 159.258 117.658) (width 0.25) (layer "F.Cu") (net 42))
 (segment (start 161.798 113.698) (end 161.798 119.126) (width 0.25) (layer "F.Cu") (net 43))
 (segment (start 161.6 113.5) (end 161.798 113.698) (width 0.25) (layer "F.Cu") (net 43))
 (segment (start 161.6 113.5) (end 125.58 113.5) (width 0.25) (layer "F.Cu") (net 43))
 (segment (start 125.58 113.5) (end 115.36 103.28) (width 0.25) (layer "F.Cu") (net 43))
 (segment (start 164.338 112.862) (end 127.482 112.862) (width 0.25) (layer "F.Cu") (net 44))
 (segment (start 164.4 112.8) (end 164.338 112.862) (width 0.25) (layer "F.Cu") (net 44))
 (segment (start 164.338 112.862) (end 164.338 119.126) (width 0.25) (layer "F.Cu") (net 44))
 (segment (start 127.482 112.862) (end 117.9 103.28) (width 0.25) (layer "F.Cu") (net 44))
 (segment (start 129.36 112.2) (end 120.44 103.28) (width 0.25) (layer "F.Cu") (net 45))
 (segment (start 166.878 112.278) (end 166.878 119.126) (width 0.25) (layer "F.Cu") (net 45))
 (segment (start 166.8 112.2) (end 166.878 112.278) (width 0.25) (layer "F.Cu") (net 45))
 (segment (start 166.8 112.2) (end 129.36 112.2) (width 0.25) (layer "F.Cu") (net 45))
 (segment (start 133.84 111.6) (end 125.52 103.28) (width 0.25) (layer "F.Cu") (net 46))
 (segment (start 168.5 111.6) (end 169.418 112.518) (width 0.25) (layer "F.Cu") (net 46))
 (segment (start 168.5 111.6) (end 133.84 111.6) (width 0.25) (layer "F.Cu") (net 46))
 (segment (start 169.418 112.518) (end 169.418 119.126) (width 0.25) (layer "F.Cu") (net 46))
 (segment (start 169.798283 119.126) (end 169.418 119.126) (width 0.25) (layer "B.Cu") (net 46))
 (segment (start 168.435717 110.9) (end 135.68 110.9) (width 0.25) (layer "F.Cu") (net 47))
 (segment (start 168.435717 110.9) (end 171.958 114.422283) (width 0.25) (layer "F.Cu") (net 47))
 (segment (start 171.958 114.422283) (end 171.958 119.126) (width 0.25) (layer "F.Cu") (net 47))
 (segment (start 135.68 110.9) (end 128.06 103.28) (width 0.25) (layer "F.Cu") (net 47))
 (segment (start 168.621914 110.45048) (end 177.038 118.866566) (width 0.25) (layer "F.Cu") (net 48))
 (segment (start 137.77048 110.45048) (end 168.621914 110.45048) (width 0.25) (layer "F.Cu") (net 48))
 (segment (start 177.038 118.866566) (end 177.038 119.126) (width 0.25) (layer "F.Cu") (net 48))
 (segment (start 130.6 103.28) (end 137.77048 110.45048) (width 0.25) (layer "F.Cu") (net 48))
 (segment (start 139.86096 110.00096) (end 170.45296 110.00096) (width 0.25) (layer "F.Cu") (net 49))
 (segment (start 133.14 103.28) (end 139.86096 110.00096) (width 0.25) (layer "F.Cu") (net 49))
 (segment (start 170.45296 110.00096) (end 179.578 119.126) (width 0.25) (layer "F.Cu") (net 49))
 (segment (start 138.22 103.28) (end 144.49144 109.55144) (width 0.25) (layer "F.Cu") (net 50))
 (segment (start 172.54344 109.55144) (end 182.118 119.126) (width 0.25) (layer "F.Cu") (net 50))
 (segment (start 144.49144 109.55144) (end 172.54344 109.55144) (width 0.25) (layer "F.Cu") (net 50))
 (segment (start 146.58192 109.10192) (end 174.63392 109.10192) (width 0.25) (layer "F.Cu") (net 51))
 (segment (start 140.76 103.28) (end 146.58192 109.10192) (width 0.25) (layer "F.Cu") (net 51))
 (segment (start 174.63392 109.10192) (end 184.658 119.126) (width 0.25) (layer "F.Cu") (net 51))
 (segment (start 148.6724 108.6524) (end 176.7244 108.6524) (width 0.25) (layer "F.Cu") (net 52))
 (segment (start 176.7244 108.6524) (end 187.198 119.126) (width 0.25) (layer "F.Cu") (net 52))
 (segment (start 143.3 103.28) (end 148.6724 108.6524) (width 0.25) (layer "F.Cu") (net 52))
 (segment (start 145.84 103.28) (end 150.76288 108.20288) (width 0.25) (layer "F.Cu") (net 53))
 (segment (start 150.76288 108.20288) (end 178.81488 108.20288) (width 0.25) (layer "F.Cu") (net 53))
 (segment (start 178.81488 108.20288) (end 189.738 119.126) (width 0.25) (layer "F.Cu") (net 53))
 (segment (start 155.39336 107.75336) (end 180.90536 107.75336) (width 0.25) (layer "F.Cu") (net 54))
 (segment (start 150.92 103.28) (end 155.39336 107.75336) (width 0.25) (layer "F.Cu") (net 54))
 (segment (start 180.90536 107.75336) (end 192.278 119.126) (width 0.25) (layer "F.Cu") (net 54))
 (segment (start 182.99584 107.30384) (end 194.818 119.126) (width 0.25) (layer "F.Cu") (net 55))
 (segment (start 153.46 103.28) (end 157.48384 107.30384) (width 0.25) (layer "F.Cu") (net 55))
 (segment (start 157.48384 107.30384) (end 182.99584 107.30384) (width 0.25) (layer "F.Cu") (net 55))
 (segment (start 145.84 85.5) (end 145.84 80.44) (width 0.25) (layer "F.Cu") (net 59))
 (segment (start 145.84 80.44) (end 142.494 77.094) (width 0.25) (layer "F.Cu") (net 59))
 (segment (start 142.494 77.094) (end 142.494 70.866) (width 0.25) (layer "F.Cu") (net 59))
 (segment (start 144.9 73.8) (end 145.034 73.666) (width 0.25) (layer "F.Cu") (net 60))
 (segment (start 150.92 79.82) (end 144.9 73.8) (width 0.25) (layer "F.Cu") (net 60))
 (segment (start 150.92 85.5) (end 150.92 79.82) (width 0.25) (layer "F.Cu") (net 60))
 (segment (start 145.034 73.666) (end 145.034 70.866) (width 0.25) (layer "F.Cu") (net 60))
 (segment (start 117.3 90.6) (end 115.4 88.7) (width 0.75) (layer "B.Cu") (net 38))
 (segment (start 138.938 119.126) (end 151.064 107) (width 0.75) (layer "B.Cu") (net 38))
 (segment (start 158 106.5) (end 158 101.5) (width 0.75) (layer "B.Cu") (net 38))
 (segment (start 151.064 107) (end 157.5 107) (width 0.75) (layer "B.Cu") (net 38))
 (segment (start 115.4 88.7) (end 115.36 88.66) (width 0.25) (layer "B.Cu") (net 38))
 (segment (start 147.1 90.6) (end 117.3 90.6) (width 0.75) (layer "B.Cu") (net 38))
 (segment (start 158 101.5) (end 147.1 90.6) (width 0.75) (layer "B.Cu") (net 38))
 (segment (start 157.5 107) (end 158 106.5) (width 0.5) (layer "B.Cu") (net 38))
 (segment (start 115.36 88.66) (end 115.36 85.5) (width 0.75) (layer "B.Cu") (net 38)))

